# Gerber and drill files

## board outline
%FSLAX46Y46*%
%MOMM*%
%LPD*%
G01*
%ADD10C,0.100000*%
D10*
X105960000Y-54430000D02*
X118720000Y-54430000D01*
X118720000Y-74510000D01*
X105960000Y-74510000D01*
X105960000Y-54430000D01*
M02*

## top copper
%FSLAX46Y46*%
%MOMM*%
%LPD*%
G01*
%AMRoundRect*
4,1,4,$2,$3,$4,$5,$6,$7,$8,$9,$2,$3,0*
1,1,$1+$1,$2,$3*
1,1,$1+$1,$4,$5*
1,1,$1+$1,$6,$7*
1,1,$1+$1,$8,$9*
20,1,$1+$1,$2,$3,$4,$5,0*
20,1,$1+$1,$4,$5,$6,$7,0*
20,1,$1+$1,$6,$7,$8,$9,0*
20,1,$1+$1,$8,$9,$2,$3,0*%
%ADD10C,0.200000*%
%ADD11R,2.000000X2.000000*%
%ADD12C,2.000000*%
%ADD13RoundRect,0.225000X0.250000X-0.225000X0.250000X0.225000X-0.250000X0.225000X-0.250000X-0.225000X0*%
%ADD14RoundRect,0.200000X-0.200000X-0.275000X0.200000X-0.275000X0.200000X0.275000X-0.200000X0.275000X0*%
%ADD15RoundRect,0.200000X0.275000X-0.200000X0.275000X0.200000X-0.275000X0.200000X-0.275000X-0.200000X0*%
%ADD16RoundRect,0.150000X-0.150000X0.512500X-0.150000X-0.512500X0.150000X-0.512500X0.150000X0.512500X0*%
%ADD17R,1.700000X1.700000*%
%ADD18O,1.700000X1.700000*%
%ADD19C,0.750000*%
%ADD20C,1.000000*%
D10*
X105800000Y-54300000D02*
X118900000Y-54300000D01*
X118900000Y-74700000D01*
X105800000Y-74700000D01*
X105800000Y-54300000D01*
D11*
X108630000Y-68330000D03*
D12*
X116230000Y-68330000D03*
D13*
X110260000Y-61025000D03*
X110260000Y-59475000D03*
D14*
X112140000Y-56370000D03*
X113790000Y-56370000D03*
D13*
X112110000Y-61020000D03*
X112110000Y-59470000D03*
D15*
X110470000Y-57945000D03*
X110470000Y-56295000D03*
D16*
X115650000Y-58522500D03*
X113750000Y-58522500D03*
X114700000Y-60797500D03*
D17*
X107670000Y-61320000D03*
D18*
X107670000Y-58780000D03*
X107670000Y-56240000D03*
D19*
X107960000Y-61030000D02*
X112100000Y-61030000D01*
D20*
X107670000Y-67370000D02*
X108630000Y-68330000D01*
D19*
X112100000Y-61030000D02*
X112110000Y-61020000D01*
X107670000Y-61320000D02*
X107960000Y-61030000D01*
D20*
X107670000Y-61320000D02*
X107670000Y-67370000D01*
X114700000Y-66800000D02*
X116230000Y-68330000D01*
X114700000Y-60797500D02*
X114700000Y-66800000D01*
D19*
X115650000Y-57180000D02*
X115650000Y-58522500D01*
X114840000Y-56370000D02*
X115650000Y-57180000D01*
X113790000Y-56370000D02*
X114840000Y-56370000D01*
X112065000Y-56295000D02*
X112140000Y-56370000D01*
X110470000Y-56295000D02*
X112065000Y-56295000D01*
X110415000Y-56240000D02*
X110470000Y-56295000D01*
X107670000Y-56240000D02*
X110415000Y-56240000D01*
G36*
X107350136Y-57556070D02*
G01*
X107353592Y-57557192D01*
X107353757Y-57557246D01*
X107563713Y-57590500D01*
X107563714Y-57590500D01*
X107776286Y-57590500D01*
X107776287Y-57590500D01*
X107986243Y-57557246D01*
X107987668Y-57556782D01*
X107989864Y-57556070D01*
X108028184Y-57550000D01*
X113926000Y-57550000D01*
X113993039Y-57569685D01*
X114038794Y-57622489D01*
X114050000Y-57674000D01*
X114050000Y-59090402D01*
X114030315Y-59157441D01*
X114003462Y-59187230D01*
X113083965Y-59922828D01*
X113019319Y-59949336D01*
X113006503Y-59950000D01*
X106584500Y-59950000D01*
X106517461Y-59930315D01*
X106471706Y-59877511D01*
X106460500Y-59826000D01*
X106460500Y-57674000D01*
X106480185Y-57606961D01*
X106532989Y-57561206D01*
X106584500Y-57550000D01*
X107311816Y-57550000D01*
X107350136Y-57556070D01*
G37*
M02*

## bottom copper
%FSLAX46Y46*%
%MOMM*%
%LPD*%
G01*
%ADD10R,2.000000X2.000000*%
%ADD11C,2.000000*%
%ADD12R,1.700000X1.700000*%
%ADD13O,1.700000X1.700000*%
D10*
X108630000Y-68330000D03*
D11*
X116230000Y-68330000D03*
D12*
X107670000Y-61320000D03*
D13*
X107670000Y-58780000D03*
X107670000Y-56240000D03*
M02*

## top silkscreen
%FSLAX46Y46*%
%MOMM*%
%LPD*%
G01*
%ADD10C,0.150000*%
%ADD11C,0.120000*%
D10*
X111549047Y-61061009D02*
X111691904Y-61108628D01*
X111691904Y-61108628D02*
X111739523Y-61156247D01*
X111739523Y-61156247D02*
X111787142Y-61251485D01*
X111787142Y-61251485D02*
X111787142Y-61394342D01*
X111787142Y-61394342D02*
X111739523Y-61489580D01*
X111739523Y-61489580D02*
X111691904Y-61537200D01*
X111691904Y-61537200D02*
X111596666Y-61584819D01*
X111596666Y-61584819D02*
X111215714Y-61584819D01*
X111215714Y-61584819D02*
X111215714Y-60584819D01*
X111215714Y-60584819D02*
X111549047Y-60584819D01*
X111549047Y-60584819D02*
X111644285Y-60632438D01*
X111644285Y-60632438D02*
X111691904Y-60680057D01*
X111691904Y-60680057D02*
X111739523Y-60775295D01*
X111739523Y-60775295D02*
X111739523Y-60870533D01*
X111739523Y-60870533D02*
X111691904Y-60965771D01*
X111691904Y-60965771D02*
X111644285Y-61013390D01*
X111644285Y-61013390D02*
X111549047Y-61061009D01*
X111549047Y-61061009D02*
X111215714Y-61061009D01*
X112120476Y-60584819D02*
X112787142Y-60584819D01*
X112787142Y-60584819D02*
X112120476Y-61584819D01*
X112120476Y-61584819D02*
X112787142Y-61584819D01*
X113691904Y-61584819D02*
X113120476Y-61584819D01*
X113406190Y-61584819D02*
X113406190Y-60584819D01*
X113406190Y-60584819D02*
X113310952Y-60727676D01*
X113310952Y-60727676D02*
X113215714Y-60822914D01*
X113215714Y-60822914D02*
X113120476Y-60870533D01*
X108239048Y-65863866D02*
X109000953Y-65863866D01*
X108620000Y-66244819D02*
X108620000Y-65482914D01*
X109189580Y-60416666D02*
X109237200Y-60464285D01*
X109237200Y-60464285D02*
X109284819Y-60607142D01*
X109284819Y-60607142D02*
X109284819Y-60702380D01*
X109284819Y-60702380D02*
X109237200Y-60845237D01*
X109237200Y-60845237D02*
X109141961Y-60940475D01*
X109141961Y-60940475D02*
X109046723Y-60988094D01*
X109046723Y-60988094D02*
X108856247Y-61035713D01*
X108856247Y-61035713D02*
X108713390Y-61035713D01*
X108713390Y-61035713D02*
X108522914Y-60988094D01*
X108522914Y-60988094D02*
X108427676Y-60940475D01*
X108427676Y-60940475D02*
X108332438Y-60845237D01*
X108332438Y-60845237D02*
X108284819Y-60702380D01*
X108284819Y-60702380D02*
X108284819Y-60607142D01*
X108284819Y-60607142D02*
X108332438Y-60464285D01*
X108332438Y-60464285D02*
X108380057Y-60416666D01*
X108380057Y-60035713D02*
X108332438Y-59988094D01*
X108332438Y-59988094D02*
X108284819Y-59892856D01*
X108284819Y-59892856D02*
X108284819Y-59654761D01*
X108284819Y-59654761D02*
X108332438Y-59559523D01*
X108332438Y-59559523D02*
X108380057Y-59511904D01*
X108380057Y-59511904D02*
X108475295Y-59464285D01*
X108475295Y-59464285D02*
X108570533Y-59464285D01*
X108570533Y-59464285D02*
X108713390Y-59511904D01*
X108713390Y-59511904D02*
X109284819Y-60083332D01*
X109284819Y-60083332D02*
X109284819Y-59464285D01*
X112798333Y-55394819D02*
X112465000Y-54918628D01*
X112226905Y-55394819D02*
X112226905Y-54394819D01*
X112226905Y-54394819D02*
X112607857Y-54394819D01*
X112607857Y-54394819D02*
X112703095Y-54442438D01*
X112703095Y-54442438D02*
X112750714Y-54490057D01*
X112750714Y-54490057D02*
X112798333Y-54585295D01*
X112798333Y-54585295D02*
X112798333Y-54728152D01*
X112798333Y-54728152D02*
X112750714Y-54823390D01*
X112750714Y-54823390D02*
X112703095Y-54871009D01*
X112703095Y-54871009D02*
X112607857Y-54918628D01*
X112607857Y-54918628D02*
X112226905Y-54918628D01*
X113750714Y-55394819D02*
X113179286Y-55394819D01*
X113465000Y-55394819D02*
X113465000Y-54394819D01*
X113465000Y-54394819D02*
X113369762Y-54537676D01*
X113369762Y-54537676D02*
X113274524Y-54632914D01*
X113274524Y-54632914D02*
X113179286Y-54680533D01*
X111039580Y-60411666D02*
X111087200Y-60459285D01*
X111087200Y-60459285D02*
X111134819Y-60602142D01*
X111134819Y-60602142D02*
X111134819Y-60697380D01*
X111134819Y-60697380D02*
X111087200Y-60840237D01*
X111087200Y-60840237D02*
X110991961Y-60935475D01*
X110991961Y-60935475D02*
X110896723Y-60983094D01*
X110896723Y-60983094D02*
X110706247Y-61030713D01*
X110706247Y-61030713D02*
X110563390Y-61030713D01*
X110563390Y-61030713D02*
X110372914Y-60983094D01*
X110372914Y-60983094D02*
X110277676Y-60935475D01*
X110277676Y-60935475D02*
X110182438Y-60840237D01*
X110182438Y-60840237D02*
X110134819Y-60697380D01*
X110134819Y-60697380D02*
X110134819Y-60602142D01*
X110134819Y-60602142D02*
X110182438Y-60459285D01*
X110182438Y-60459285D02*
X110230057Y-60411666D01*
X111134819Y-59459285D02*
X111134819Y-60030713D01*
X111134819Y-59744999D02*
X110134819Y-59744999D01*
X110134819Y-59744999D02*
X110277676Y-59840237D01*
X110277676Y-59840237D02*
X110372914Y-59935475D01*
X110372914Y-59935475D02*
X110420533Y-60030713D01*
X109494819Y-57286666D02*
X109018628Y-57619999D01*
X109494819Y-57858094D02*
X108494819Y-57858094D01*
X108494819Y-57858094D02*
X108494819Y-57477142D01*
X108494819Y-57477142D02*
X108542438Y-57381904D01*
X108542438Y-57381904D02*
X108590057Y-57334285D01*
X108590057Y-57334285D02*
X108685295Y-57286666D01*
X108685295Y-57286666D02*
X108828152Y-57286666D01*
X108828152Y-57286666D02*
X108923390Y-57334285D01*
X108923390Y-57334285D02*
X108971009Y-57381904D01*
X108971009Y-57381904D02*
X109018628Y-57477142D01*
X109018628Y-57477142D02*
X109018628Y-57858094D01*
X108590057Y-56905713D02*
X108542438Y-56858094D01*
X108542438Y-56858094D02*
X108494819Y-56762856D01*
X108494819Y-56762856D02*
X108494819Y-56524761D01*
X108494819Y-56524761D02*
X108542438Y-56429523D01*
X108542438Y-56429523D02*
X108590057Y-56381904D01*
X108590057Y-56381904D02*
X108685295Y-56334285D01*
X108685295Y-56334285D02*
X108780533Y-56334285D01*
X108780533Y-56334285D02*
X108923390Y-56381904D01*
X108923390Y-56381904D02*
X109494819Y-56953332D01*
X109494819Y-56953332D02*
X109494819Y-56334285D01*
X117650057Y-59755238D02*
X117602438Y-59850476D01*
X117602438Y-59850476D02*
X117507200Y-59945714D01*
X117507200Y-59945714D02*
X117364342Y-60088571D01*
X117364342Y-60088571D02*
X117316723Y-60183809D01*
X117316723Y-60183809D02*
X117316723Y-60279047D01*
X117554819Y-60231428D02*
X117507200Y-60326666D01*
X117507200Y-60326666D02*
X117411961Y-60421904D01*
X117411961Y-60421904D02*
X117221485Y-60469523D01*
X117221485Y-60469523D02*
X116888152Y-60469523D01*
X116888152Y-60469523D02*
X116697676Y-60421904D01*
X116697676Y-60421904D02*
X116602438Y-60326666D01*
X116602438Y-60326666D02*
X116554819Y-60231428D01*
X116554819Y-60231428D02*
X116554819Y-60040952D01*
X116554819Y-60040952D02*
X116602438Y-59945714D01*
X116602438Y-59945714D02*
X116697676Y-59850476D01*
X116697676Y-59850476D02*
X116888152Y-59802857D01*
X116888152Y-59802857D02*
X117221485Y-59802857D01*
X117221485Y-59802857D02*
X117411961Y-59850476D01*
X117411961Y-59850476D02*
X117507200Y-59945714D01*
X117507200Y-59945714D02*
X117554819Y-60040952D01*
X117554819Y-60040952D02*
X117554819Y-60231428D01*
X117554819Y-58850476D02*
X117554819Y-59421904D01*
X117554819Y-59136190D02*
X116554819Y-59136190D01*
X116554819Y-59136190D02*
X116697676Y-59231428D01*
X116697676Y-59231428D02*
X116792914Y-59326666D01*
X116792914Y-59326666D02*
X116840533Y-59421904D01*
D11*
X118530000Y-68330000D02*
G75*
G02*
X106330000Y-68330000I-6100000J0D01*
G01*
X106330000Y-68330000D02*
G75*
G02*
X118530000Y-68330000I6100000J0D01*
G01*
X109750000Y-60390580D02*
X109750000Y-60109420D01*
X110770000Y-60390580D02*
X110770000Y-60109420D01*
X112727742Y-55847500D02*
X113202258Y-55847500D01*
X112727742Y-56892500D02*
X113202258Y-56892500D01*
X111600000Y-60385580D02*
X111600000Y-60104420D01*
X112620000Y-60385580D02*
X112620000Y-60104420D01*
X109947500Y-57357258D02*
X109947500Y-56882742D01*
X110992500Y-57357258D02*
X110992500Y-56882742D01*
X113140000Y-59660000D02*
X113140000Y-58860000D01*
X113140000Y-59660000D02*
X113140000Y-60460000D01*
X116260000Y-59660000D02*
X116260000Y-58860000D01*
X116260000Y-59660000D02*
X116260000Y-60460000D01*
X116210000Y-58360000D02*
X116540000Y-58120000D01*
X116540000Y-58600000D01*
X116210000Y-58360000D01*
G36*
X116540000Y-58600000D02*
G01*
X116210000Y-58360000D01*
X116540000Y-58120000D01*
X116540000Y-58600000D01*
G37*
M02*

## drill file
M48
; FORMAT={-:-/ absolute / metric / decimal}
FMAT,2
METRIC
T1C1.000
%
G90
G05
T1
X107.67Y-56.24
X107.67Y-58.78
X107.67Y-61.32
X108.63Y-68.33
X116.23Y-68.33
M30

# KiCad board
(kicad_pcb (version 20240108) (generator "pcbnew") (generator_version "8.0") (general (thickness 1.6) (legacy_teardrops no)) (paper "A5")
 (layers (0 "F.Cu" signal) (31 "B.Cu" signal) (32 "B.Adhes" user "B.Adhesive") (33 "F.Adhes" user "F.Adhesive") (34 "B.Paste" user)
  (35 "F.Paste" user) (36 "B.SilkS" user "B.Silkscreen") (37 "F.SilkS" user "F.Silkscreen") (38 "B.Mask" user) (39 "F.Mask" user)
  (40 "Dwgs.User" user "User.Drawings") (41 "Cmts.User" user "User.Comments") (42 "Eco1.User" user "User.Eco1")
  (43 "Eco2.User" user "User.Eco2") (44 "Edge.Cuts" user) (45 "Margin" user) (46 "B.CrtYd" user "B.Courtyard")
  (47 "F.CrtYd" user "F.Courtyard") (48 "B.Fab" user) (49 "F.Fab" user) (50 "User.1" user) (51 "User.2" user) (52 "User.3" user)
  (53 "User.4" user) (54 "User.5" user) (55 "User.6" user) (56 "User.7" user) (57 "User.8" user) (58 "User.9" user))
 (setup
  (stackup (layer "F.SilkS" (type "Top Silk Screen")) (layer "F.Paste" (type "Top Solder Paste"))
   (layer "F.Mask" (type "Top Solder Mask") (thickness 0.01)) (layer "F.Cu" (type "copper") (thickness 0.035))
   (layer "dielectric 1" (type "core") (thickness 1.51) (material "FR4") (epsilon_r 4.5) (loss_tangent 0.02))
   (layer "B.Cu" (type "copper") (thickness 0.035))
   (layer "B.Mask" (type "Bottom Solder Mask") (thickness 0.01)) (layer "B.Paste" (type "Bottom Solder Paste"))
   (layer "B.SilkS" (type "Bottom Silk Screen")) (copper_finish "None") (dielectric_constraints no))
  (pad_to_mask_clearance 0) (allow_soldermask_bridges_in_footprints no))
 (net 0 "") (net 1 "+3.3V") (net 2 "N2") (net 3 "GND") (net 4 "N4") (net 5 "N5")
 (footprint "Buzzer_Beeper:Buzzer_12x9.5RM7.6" (layer "F.Cu") (at 108.63 68.33)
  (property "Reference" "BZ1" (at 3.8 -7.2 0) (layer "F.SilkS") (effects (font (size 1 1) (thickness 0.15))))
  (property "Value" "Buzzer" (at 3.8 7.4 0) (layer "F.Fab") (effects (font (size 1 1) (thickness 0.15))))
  (fp_circle (center 3.8 0) (end 9.9 0) (stroke (width 0.12) (type solid)) (fill none) (layer "F.SilkS"))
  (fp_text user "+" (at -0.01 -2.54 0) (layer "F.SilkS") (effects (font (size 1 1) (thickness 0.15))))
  (pad "1" thru_hole rect (at 0 0) (size 2 2) (drill 1) (layers "*.Cu" "*.Mask") (remove_unused_layers no) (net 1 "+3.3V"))
  (pad "2" thru_hole circle (at 7.6 0) (size 2 2) (drill 1) (layers "*.Cu" "*.Mask") (remove_unused_layers no) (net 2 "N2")))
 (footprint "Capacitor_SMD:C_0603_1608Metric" (layer "F.Cu") (at 110.26 60.25 90)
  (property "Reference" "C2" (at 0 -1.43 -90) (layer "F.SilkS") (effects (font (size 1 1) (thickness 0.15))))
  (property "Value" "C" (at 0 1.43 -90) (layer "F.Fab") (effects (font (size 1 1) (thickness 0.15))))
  (fp_line (start -0.14058 -0.51) (end 0.14058 -0.51) (stroke (width 0.12) (type solid)) (layer "F.SilkS"))
  (fp_line (start -0.14058 0.51) (end 0.14058 0.51) (stroke (width 0.12) (type solid)) (layer "F.SilkS"))
  (pad "1" smd roundrect (at -0.775 0 90) (size 0.9 0.95) (layers "F.Cu" "F.Paste" "F.Mask") (roundrect_rratio 0.25) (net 1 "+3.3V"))
  (pad "2" smd roundrect (at 0.775 0 90) (size 0.9 0.95) (layers "F.Cu" "F.Paste" "F.Mask") (roundrect_rratio 0.25) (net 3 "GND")))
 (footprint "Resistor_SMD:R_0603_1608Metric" (layer "F.Cu") (at 112.965 56.37)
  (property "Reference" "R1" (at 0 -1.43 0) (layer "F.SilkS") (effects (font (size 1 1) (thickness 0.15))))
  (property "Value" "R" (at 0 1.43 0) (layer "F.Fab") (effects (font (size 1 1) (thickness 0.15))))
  (fp_line (start -0.237258 -0.5225) (end 0.237258 -0.5225) (stroke (width 0.12) (type solid)) (layer "F.SilkS"))
  (fp_line (start -0.237258 0.5225) (end 0.237258 0.5225) (stroke (width 0.12) (type solid)) (layer "F.SilkS"))
  (pad "1" smd roundrect (at -0.825 0) (size 0.8 0.95) (layers "F.Cu" "F.Paste" "F.Mask") (roundrect_rratio 0.25) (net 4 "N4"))
  (pad "2" smd roundrect (at 0.825 0) (size 0.8 0.95) (layers "F.Cu" "F.Paste" "F.Mask") (roundrect_rratio 0.25) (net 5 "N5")))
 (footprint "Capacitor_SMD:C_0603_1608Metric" (layer "F.Cu") (at 112.11 60.245 90)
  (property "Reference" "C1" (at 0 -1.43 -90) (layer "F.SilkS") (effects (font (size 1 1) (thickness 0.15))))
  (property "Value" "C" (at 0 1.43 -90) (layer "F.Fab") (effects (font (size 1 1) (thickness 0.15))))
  (fp_line (start -0.14058 -0.51) (end 0.14058 -0.51) (stroke (width 0.12) (type solid)) (layer "F.SilkS"))
  (fp_line (start -0.14058 0.51) (end 0.14058 0.51) (stroke (width 0.12) (type solid)) (layer "F.SilkS"))
  (pad "1" smd roundrect (at -0.775 0 90) (size 0.9 0.95) (layers "F.Cu" "F.Paste" "F.Mask") (roundrect_rratio 0.25) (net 1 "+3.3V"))
  (pad "2" smd roundrect (at 0.775 0 90) (size 0.9 0.95) (layers "F.Cu" "F.Paste" "F.Mask") (roundrect_rratio 0.25) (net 3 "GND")))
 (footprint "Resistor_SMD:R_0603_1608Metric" (layer "F.Cu") (at 110.47 57.12 90)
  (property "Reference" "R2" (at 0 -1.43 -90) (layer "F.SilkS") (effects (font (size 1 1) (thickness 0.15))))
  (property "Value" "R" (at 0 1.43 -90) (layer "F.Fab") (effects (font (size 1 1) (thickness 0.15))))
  (fp_line (start -0.237258 -0.5225) (end 0.237258 -0.5225) (stroke (width 0.12) (type solid)) (layer "F.SilkS"))
  (fp_line (start -0.237258 0.5225) (end 0.237258 0.5225) (stroke (width 0.12) (type solid)) (layer "F.SilkS"))
  (pad "1" smd roundrect (at -0.825 0 90) (size 0.8 0.95) (layers "F.Cu" "F.Paste" "F.Mask") (roundrect_rratio 0.25) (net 3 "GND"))
  (pad "2" smd roundrect (at 0.825 0 90) (size 0.8 0.95) (layers "F.Cu" "F.Paste" "F.Mask") (roundrect_rratio 0.25) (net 4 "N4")))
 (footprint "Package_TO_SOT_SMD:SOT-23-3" (layer "F.Cu") (at 114.7 59.66 -90)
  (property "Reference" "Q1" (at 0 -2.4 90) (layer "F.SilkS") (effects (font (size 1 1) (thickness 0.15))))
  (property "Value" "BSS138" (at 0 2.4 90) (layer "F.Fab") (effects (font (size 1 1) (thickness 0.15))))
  (fp_line (start 0 1.56) (end -0.8 1.56) (stroke (width 0.12) (type solid)) (layer "F.SilkS"))
  (fp_line (start 0 1.56) (end 0.8 1.56) (stroke (width 0.12) (type solid)) (layer "F.SilkS"))
  (fp_line (start 0 -1.56) (end -0.8 -1.56) (stroke (width 0.12) (type solid)) (layer "F.SilkS"))
  (fp_line (start 0 -1.56) (end 0.8 -1.56) (stroke (width 0.12) (type solid)) (layer "F.SilkS"))
  (fp_poly
   (pts (xy -1.3 -1.51) (xy -1.54 -1.84) (xy -1.06 -1.84) (xy -1.3 -1.51)) (stroke (width 0.12) (type solid)) (fill solid) (layer "F.SilkS"))
  (pad "1" smd roundrect (at -1.1375 -0.95 270) (size 1.325 0.6) (layers "F.Cu" "F.Paste" "F.Mask") (roundrect_rratio 0.25) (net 5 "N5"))
  (pad "2" smd roundrect (at -1.1375 0.95 270) (size 1.325 0.6) (layers "F.Cu" "F.Paste" "F.Mask") (roundrect_rratio 0.25) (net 3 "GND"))
  (pad "3" smd roundrect (at 1.1375 0 270) (size 1.325 0.6) (layers "F.Cu" "F.Paste" "F.Mask") (roundrect_rratio 0.25) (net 2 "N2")))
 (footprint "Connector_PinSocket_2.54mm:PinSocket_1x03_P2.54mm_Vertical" (layer "B.Cu") (at 107.67 61.32)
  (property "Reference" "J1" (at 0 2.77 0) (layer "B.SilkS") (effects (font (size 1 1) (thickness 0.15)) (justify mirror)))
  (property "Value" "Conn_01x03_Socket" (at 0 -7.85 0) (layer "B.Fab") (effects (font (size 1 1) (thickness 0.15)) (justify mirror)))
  (pad "1" thru_hole rect (at 0 0) (size 1.7 1.7) (drill 1) (layers "*.Cu" "*.Mask") (remove_unused_layers no) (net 1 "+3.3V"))
  (pad "2" thru_hole oval (at 0 -2.54) (size 1.7 1.7) (drill 1) (layers "*.Cu" "*.Mask") (remove_unused_layers no) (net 3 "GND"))
  (pad "3" thru_hole oval (at 0 -5.08) (size 1.7 1.7) (drill 1) (layers "*.Cu" "*.Mask") (remove_unused_layers no) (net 4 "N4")))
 (gr_rect (start 105.8 54.3) (end 118.9 74.7) (stroke (width 0.2) (type default)) (fill none) (layer "F.Cu"))
 (gr_rect (start 105.96 54.43) (end 118.72 74.51) (stroke (width 0.1) (type default)) (fill none) (layer "Edge.Cuts"))
 (segment (start 107.96 61.03) (end 112.1 61.03) (width 0.75) (layer "F.Cu") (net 1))
 (segment (start 107.67 67.37) (end 108.63 68.33) (width 1) (layer "F.Cu") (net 1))
 (segment (start 112.1 61.03) (end 112.11 61.02) (width 0.75) (layer "F.Cu") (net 1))
 (segment (start 107.67 61.32) (end 107.96 61.03) (width 0.75) (layer "F.Cu") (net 1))
 (segment (start 107.67 61.32) (end 107.67 67.37) (width 1) (layer "F.Cu") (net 1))
 (segment (start 114.7 66.8) (end 116.23 68.33) (width 1) (layer "F.Cu") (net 2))
 (segment (start 114.7 60.7975) (end 114.7 66.8) (width 1) (layer "F.Cu") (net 2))
 (segment (start 115.65 57.18) (end 115.65 58.5225) (width 0.75) (layer "F.Cu") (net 5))
 (segment (start 114.84 56.37) (end 115.65 57.18) (width 0.75) (layer "F.Cu") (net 5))
 (segment (start 113.79 56.37) (end 114.84 56.37) (width 0.75) (layer "F.Cu") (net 5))
 (segment (start 112.065 56.295) (end 112.14 56.37) (width 0.75) (layer "F.Cu") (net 4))
 (segment (start 110.47 56.295) (end 112.065 56.295) (width 0.75) (layer "F.Cu") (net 4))
 (segment (start 110.415 56.24) (end 110.47 56.295) (width 0.75) (layer "F.Cu") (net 4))
 (segment (start 107.67 56.24) (end 110.415 56.24) (width 0.75) (layer "F.Cu") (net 4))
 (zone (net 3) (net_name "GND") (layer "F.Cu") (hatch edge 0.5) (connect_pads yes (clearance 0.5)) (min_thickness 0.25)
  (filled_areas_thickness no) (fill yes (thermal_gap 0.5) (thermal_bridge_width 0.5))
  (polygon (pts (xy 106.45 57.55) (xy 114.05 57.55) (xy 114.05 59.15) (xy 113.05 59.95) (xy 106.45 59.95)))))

